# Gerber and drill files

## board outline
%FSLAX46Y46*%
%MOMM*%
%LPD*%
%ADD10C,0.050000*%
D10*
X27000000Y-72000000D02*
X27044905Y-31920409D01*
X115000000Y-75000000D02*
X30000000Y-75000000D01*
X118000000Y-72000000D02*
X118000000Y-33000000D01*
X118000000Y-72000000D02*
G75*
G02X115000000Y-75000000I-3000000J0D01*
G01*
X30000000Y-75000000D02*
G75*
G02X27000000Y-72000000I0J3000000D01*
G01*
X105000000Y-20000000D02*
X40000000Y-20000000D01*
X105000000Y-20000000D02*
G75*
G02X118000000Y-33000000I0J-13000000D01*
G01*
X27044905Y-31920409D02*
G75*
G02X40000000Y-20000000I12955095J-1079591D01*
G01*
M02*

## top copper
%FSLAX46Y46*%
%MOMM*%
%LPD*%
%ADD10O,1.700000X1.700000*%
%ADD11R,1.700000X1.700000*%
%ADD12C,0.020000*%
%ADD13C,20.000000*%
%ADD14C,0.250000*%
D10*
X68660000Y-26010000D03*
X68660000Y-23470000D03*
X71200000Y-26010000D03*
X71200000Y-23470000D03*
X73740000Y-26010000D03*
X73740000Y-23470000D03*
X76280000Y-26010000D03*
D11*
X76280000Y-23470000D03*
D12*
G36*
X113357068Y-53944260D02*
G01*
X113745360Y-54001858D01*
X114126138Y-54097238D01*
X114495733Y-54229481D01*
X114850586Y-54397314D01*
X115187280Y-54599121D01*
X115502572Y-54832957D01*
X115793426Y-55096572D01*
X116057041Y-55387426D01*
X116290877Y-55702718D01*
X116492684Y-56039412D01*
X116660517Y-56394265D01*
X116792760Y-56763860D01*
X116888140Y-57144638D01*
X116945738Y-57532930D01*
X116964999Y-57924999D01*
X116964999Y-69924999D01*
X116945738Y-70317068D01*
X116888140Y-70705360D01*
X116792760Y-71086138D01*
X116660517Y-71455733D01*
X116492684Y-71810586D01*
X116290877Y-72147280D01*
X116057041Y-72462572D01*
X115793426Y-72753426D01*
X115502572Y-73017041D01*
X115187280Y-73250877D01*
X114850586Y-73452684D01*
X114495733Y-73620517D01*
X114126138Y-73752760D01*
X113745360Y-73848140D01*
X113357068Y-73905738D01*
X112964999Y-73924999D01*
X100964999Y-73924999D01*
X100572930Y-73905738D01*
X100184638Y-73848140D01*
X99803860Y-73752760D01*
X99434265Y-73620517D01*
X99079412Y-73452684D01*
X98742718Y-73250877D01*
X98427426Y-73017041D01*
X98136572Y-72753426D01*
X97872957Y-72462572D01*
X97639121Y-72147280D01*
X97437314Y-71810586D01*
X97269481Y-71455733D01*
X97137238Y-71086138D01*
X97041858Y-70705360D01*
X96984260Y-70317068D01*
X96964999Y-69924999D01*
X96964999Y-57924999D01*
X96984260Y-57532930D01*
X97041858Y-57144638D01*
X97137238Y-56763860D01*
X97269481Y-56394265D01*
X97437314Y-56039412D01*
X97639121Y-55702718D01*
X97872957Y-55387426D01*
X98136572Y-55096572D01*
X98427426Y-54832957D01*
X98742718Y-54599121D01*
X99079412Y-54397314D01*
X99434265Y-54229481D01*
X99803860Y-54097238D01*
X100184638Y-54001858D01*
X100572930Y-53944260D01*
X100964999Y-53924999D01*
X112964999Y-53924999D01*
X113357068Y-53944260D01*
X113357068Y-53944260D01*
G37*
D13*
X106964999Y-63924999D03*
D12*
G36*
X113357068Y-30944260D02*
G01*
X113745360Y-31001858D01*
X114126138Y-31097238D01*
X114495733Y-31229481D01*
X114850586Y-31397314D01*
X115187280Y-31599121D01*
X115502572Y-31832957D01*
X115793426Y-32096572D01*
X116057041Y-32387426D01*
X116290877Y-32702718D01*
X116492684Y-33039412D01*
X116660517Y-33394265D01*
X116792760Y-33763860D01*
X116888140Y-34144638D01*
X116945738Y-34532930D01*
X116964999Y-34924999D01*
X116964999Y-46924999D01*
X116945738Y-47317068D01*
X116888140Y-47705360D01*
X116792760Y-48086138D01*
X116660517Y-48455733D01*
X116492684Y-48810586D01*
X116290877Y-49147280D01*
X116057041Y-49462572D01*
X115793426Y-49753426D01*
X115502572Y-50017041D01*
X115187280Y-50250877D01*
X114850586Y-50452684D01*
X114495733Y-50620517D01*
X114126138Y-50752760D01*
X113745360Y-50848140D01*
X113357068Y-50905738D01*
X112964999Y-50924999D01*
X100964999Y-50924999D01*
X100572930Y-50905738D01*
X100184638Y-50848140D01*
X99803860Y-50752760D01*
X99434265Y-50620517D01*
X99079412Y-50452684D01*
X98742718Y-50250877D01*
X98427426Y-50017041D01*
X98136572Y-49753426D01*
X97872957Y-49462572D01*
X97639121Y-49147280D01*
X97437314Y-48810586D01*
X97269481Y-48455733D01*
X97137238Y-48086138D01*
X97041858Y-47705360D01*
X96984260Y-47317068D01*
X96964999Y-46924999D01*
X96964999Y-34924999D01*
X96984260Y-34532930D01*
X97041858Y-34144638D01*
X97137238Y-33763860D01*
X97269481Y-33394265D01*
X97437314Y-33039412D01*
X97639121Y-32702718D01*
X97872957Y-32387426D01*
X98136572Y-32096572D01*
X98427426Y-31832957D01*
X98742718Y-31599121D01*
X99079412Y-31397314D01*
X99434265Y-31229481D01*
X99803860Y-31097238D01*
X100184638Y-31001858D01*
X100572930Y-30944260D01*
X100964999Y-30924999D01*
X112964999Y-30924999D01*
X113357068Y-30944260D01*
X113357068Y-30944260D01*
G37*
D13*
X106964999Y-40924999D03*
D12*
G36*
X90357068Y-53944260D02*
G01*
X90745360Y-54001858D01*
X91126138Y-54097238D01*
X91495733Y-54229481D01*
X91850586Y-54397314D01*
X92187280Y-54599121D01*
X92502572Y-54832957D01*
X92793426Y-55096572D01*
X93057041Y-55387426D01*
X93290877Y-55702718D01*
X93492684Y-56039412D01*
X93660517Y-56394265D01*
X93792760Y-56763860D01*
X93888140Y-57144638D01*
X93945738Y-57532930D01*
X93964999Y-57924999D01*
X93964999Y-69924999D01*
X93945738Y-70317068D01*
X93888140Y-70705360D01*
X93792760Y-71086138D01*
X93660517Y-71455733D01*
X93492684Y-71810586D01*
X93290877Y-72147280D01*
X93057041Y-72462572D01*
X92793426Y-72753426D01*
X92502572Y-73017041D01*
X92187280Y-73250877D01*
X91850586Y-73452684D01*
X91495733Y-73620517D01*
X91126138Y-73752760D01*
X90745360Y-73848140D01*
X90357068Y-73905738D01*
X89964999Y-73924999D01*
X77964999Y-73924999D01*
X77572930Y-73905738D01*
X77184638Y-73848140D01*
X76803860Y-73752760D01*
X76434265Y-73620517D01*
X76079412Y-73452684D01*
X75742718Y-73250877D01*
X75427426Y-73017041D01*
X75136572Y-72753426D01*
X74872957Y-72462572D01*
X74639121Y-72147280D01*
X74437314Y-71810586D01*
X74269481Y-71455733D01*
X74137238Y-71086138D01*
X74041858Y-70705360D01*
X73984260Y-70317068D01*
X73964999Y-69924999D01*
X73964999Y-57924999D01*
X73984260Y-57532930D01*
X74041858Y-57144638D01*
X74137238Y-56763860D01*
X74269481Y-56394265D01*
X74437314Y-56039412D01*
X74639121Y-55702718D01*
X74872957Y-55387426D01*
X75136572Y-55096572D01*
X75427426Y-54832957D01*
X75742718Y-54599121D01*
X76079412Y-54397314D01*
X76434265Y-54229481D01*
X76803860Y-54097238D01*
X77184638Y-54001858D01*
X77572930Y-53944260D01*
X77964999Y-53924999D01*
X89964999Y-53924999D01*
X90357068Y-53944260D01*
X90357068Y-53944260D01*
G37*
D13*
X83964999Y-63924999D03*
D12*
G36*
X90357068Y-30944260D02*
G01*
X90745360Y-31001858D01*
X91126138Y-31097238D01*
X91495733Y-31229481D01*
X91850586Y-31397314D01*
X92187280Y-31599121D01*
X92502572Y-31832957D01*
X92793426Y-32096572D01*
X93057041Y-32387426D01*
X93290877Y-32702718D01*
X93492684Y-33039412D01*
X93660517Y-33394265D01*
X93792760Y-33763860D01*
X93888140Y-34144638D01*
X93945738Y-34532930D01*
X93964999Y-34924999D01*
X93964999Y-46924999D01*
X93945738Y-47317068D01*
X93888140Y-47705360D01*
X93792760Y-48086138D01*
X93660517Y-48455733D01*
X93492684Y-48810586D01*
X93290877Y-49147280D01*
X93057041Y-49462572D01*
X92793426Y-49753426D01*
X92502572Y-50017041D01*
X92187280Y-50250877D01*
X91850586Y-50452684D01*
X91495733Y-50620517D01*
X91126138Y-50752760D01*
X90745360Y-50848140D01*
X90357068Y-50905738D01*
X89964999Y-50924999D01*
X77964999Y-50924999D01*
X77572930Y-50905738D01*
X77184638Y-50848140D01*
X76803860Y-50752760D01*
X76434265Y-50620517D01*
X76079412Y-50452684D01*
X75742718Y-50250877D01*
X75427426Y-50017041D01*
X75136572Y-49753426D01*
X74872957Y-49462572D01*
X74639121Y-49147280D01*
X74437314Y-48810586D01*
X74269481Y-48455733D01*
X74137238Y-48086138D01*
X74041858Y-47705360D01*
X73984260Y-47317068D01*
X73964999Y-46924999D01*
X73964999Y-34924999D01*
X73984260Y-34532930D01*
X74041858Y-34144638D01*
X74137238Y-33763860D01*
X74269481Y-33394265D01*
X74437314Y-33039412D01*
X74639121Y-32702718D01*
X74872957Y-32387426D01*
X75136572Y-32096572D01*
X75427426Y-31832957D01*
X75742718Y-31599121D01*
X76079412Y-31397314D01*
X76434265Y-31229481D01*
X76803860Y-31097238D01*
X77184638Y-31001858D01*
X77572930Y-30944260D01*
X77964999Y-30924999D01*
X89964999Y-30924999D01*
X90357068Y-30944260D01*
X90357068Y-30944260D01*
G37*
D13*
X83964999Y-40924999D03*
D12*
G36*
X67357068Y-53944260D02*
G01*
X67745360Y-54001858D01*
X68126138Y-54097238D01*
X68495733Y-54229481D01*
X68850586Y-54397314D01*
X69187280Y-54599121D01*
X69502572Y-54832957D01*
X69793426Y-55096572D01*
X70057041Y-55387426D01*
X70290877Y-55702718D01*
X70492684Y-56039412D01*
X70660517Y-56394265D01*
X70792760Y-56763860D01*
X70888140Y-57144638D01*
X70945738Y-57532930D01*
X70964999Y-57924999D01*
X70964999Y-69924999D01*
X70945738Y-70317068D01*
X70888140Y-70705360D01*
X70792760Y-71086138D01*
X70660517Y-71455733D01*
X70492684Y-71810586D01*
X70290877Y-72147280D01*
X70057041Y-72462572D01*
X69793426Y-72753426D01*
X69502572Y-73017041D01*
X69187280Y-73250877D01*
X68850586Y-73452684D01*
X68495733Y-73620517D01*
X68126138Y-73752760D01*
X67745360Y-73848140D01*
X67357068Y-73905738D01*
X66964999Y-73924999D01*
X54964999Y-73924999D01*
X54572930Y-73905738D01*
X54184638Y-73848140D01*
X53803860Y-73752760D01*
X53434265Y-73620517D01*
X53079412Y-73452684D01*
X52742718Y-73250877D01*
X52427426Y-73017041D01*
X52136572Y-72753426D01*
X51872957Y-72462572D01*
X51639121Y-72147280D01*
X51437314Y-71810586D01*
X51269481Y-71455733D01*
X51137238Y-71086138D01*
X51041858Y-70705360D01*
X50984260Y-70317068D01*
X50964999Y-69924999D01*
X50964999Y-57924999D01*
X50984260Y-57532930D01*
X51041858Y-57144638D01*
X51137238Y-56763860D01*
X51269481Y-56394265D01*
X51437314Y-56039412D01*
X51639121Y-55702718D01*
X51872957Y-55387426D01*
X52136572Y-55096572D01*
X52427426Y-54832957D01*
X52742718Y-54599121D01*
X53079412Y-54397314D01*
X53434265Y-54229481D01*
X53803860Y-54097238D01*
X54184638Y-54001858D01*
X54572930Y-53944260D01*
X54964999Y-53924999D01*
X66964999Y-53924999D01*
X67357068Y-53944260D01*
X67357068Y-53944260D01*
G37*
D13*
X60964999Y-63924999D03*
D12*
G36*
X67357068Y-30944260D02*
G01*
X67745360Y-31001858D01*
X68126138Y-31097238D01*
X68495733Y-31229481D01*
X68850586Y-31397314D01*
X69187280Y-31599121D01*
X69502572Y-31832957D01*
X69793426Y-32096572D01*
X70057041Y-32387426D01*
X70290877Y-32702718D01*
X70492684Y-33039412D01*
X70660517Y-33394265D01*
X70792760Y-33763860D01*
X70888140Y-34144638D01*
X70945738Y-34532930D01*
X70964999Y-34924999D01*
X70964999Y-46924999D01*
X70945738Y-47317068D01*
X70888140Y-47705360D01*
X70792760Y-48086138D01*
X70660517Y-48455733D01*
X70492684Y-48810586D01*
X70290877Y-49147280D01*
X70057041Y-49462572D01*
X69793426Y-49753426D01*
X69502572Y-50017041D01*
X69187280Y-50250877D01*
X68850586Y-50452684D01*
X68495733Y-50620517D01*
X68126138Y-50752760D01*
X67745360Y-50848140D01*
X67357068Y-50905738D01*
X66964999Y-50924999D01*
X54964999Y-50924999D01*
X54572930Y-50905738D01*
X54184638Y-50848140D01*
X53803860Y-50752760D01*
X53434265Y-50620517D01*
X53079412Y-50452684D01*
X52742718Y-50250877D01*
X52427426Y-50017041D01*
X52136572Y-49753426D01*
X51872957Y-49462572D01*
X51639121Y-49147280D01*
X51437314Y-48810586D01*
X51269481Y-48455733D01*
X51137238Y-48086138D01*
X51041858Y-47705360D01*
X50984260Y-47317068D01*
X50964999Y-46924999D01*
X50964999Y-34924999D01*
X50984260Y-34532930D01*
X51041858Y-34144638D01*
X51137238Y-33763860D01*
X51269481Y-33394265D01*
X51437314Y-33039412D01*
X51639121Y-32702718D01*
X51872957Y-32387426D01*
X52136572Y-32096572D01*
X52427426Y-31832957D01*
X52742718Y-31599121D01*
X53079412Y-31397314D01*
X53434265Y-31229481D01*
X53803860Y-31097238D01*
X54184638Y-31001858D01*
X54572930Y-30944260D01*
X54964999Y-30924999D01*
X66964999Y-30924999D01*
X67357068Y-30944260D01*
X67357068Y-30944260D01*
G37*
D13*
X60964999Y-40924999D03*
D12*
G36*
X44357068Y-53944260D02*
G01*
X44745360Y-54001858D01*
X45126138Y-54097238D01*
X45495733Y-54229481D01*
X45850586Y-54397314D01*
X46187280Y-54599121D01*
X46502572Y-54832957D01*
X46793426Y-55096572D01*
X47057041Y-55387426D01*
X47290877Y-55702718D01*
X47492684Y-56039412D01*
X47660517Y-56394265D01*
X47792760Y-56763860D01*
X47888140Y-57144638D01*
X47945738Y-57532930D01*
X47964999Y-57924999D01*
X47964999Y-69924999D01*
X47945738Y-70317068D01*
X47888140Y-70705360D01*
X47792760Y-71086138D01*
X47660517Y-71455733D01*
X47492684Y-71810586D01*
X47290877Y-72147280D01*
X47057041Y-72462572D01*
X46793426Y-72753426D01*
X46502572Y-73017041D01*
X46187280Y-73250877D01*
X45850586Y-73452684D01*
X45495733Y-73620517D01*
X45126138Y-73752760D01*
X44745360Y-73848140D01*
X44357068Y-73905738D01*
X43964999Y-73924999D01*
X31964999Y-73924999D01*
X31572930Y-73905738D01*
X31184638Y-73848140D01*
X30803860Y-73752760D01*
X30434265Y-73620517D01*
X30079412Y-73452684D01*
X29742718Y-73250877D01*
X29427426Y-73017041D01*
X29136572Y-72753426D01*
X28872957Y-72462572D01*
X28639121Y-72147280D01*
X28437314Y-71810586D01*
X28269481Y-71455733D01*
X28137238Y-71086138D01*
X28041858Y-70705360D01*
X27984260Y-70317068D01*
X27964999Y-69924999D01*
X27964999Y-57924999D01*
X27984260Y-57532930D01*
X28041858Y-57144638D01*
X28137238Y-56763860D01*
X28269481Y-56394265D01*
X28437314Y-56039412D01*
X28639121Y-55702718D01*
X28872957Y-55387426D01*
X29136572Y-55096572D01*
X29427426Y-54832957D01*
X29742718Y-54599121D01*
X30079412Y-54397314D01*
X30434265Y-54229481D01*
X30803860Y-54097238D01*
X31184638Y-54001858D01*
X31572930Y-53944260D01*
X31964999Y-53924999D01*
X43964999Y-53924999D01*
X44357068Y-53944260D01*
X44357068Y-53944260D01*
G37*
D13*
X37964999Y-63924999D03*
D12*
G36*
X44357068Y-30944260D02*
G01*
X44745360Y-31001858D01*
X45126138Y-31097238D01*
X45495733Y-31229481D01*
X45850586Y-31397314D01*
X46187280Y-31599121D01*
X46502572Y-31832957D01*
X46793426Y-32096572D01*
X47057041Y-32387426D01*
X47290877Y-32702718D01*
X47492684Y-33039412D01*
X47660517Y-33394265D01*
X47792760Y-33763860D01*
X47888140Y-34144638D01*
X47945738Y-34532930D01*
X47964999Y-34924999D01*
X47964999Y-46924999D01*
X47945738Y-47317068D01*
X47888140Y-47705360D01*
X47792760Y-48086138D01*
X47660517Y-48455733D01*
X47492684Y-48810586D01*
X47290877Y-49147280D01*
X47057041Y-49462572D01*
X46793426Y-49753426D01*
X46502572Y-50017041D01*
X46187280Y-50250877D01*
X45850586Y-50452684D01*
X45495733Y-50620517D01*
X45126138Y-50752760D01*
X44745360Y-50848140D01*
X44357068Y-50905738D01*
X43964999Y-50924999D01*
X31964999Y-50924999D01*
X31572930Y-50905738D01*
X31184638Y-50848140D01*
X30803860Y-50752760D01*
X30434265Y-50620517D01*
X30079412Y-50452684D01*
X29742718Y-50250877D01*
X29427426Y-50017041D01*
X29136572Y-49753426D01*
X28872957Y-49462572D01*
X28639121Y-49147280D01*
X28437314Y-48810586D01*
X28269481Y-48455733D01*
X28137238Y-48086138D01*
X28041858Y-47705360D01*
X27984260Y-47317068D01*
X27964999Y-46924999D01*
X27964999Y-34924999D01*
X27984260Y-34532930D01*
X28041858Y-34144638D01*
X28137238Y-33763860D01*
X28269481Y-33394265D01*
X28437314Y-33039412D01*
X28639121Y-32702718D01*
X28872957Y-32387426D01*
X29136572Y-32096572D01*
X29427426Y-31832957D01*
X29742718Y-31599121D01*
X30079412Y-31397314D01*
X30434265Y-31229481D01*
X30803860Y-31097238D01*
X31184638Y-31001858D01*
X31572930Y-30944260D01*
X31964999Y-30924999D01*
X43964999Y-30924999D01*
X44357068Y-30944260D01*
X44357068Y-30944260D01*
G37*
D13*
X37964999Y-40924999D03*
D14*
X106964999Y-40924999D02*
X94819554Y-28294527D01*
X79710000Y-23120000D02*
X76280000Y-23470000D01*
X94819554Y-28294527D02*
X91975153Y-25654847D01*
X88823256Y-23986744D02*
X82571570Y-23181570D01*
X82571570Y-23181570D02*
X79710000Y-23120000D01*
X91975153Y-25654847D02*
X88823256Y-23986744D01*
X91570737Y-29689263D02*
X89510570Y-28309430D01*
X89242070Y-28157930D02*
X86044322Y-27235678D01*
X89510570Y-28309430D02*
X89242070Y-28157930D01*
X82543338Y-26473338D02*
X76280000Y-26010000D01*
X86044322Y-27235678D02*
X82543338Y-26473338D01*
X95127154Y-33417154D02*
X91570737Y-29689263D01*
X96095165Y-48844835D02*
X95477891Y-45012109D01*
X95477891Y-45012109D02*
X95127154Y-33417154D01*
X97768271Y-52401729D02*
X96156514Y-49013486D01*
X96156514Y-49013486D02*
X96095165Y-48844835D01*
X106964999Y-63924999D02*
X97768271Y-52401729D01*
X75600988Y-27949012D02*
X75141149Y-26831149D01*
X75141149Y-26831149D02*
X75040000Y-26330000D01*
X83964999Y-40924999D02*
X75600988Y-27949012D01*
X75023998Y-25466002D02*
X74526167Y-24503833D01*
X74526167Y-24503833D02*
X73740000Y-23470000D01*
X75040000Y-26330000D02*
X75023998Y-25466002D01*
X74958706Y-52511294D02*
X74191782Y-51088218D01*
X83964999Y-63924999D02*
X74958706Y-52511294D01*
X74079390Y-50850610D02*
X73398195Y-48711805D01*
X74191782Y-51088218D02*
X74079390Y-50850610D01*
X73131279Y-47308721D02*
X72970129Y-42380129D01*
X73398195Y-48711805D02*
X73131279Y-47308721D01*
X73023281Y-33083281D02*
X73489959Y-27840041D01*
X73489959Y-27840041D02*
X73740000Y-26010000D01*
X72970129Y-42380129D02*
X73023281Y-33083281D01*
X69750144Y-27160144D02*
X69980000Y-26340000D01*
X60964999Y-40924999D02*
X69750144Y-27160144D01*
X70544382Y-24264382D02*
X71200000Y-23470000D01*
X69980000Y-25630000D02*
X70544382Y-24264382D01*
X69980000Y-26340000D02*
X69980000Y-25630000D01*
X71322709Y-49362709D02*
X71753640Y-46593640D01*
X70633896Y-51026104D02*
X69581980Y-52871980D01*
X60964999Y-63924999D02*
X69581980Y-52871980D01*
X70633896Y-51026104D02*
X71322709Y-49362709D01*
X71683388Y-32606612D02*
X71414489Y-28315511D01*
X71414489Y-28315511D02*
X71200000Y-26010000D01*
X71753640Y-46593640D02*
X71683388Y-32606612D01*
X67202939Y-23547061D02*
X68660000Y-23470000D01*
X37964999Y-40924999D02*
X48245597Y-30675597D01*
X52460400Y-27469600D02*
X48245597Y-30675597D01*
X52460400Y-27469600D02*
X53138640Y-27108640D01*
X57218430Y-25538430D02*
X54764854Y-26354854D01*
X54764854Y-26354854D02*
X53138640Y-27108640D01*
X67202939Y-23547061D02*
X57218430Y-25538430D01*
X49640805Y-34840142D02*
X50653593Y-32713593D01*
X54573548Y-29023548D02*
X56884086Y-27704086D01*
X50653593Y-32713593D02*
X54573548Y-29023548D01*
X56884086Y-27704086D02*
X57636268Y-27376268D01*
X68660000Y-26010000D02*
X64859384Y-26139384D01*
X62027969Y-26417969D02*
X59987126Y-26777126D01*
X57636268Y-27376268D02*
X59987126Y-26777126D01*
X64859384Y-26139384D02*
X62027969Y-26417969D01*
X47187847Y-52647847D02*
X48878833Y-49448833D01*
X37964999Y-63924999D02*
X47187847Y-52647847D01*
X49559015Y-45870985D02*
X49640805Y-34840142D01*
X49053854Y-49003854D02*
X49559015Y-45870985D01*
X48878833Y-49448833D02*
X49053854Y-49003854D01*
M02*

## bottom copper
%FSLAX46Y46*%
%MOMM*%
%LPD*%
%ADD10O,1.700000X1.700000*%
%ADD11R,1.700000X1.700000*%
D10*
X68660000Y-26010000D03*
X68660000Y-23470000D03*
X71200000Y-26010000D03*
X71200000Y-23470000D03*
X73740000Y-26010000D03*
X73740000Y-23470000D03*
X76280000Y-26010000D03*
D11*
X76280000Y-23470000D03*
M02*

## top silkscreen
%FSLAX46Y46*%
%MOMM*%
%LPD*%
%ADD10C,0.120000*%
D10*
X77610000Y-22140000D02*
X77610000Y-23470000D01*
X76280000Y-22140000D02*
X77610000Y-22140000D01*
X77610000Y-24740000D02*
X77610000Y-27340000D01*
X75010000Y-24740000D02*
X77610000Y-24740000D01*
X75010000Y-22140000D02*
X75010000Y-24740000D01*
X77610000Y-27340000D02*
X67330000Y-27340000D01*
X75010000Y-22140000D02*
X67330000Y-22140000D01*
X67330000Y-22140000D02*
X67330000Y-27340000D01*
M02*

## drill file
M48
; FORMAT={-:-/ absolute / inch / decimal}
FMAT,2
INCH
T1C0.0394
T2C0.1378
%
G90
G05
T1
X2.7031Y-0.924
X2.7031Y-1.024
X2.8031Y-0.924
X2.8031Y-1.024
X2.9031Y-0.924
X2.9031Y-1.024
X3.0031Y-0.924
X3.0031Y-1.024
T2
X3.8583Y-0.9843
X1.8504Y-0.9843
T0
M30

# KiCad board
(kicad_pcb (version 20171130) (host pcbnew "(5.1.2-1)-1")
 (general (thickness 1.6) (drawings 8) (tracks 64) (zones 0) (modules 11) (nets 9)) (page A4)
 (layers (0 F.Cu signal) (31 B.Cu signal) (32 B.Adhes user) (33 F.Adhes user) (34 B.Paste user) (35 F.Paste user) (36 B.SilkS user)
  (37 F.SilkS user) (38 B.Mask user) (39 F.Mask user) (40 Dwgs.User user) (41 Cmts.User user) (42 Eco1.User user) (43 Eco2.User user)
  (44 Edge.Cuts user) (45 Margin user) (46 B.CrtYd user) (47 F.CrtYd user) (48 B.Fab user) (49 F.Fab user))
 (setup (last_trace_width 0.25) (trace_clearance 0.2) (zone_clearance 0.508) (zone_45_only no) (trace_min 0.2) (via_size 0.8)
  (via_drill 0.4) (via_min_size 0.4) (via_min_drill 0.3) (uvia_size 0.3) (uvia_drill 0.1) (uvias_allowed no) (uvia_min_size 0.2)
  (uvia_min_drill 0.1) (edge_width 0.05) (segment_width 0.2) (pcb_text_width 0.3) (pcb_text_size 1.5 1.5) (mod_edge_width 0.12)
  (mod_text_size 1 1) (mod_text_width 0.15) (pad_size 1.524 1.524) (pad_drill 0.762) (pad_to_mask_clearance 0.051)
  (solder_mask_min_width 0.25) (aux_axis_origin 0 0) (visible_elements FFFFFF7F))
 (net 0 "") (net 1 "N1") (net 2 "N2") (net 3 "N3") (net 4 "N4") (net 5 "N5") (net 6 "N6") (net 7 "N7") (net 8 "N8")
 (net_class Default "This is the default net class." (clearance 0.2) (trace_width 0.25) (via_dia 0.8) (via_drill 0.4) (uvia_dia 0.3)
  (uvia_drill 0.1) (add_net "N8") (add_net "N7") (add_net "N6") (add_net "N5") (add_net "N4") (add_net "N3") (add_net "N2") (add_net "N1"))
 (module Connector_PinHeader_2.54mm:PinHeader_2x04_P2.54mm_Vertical (layer F.Cu) (at 76.28 23.47 270)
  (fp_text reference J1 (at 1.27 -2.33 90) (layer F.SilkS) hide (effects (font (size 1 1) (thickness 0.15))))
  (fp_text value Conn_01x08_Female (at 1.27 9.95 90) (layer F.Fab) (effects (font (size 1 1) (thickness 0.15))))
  (fp_line (start -1.33 -1.33) (end 0 -1.33) (layer F.SilkS) (width 0.12))
  (fp_line (start -1.33 0) (end -1.33 -1.33) (layer F.SilkS) (width 0.12))
  (fp_line (start 1.27 -1.33) (end 3.87 -1.33) (layer F.SilkS) (width 0.12))
  (fp_line (start 1.27 1.27) (end 1.27 -1.33) (layer F.SilkS) (width 0.12))
  (fp_line (start -1.33 1.27) (end 1.27 1.27) (layer F.SilkS) (width 0.12))
  (fp_line (start 3.87 -1.33) (end 3.87 8.95) (layer F.SilkS) (width 0.12))
  (fp_line (start -1.33 1.27) (end -1.33 8.95) (layer F.SilkS) (width 0.12))
  (fp_line (start -1.33 8.95) (end 3.87 8.95) (layer F.SilkS) (width 0.12))
  (pad 8 thru_hole oval (at 2.54 7.62 270) (size 1.7 1.7) (drill 1) (layers *.Cu *.Mask) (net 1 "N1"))
  (pad 7 thru_hole oval (at 0 7.62 270) (size 1.7 1.7) (drill 1) (layers *.Cu *.Mask) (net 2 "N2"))
  (pad 6 thru_hole oval (at 2.54 5.08 270) (size 1.7 1.7) (drill 1) (layers *.Cu *.Mask) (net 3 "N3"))
  (pad 5 thru_hole oval (at 0 5.08 270) (size 1.7 1.7) (drill 1) (layers *.Cu *.Mask) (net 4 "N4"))
  (pad 4 thru_hole oval (at 2.54 2.54 270) (size 1.7 1.7) (drill 1) (layers *.Cu *.Mask) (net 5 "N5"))
  (pad 3 thru_hole oval (at 0 2.54 270) (size 1.7 1.7) (drill 1) (layers *.Cu *.Mask) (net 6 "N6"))
  (pad 2 thru_hole oval (at 2.54 0 270) (size 1.7 1.7) (drill 1) (layers *.Cu *.Mask) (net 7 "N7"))
  (pad 1 thru_hole rect (at 0 0 270) (size 1.7 1.7) (drill 1) (layers *.Cu *.Mask) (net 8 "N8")))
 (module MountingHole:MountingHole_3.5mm (layer F.Cu) (at 98 25)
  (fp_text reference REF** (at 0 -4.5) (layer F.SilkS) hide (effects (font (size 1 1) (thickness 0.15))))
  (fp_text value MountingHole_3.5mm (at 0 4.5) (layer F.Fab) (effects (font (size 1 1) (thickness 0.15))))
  (pad 1 np_thru_hole circle (at 0 0) (size 3.5 3.5) (drill 3.5) (layers *.Cu *.Mask)))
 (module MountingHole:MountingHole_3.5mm (layer F.Cu) (at 47 25)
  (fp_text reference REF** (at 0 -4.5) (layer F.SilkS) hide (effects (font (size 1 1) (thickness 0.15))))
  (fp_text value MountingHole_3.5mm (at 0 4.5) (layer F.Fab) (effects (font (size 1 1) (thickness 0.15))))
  (pad 1 np_thru_hole circle (at 0 0) (size 3.5 3.5) (drill 3.5) (layers *.Cu *.Mask)))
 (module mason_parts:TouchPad (layer F.Cu) (at 106.984999 63.964999)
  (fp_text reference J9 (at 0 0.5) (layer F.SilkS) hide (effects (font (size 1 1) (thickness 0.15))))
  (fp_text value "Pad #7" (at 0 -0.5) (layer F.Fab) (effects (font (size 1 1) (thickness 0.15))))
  (pad 1 smd roundrect (at -0.02 -0.04) (size 20 20) (layers F.Cu F.Paste F.Mask) (roundrect_rratio 0.2) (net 7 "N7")))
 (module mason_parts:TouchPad (layer F.Cu) (at 106.984999 40.964999)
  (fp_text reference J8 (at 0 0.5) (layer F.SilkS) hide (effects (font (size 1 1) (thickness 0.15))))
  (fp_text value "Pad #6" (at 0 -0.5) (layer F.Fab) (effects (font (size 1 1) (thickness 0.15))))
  (pad 1 smd roundrect (at -0.02 -0.04) (size 20 20) (layers F.Cu F.Paste F.Mask) (roundrect_rratio 0.2) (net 8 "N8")))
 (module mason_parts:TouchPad (layer F.Cu) (at 83.984999 63.964999)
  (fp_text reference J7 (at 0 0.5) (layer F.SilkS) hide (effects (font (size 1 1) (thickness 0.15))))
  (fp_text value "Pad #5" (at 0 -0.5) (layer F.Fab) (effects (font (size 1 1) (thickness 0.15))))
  (pad 1 smd roundrect (at -0.02 -0.04) (size 20 20) (layers F.Cu F.Paste F.Mask) (roundrect_rratio 0.2) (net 5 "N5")))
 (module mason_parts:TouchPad (layer F.Cu) (at 83.984999 40.964999)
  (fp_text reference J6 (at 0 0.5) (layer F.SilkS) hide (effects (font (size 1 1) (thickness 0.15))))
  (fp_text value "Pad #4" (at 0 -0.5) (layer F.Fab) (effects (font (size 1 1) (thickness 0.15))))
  (pad 1 smd roundrect (at -0.02 -0.04) (size 20 20) (layers F.Cu F.Paste F.Mask) (roundrect_rratio 0.2) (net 6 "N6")))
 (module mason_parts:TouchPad (layer F.Cu) (at 60.984999 63.964999)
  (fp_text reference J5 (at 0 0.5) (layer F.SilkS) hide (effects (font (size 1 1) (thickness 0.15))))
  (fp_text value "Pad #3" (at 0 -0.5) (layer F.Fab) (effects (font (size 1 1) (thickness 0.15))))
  (pad 1 smd roundrect (at -0.02 -0.04) (size 20 20) (layers F.Cu F.Paste F.Mask) (roundrect_rratio 0.2) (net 3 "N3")))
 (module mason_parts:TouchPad (layer F.Cu) (at 60.984999 40.964999)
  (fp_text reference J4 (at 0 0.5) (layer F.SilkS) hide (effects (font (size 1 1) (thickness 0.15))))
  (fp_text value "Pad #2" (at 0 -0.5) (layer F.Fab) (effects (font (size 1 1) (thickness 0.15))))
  (pad 1 smd roundrect (at -0.02 -0.04) (size 20 20) (layers F.Cu F.Paste F.Mask) (roundrect_rratio 0.2) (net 4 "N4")))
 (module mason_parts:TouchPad (layer F.Cu) (at 37.984999 63.964999)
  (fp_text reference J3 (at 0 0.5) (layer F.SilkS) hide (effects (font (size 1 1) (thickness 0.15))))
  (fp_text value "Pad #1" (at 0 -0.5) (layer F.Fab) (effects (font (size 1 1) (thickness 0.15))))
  (pad 1 smd roundrect (at -0.02 -0.04) (size 20 20) (layers F.Cu F.Paste F.Mask) (roundrect_rratio 0.2) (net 1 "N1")))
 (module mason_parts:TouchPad (layer F.Cu) (at 37.984999 40.964999)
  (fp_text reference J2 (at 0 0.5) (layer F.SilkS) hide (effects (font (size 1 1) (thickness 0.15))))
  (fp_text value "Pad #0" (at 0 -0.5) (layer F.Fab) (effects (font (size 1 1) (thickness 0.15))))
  (pad 1 smd roundrect (at -0.02 -0.04) (size 20 20) (layers F.Cu F.Paste F.Mask) (roundrect_rratio 0.2) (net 2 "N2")))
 (gr_line (start 27 72) (end 27.044905 31.920409) (layer Edge.Cuts) (width 0.05))
 (gr_line (start 115 75) (end 30 75) (layer Edge.Cuts) (width 0.05))
 (gr_line (start 118 72) (end 118 33) (layer Edge.Cuts) (width 0.05))
 (gr_arc (start 115 72) (end 115 75) (angle -90) (layer Edge.Cuts) (width 0.05))
 (gr_arc (start 30 72) (end 27 72) (angle -90) (layer Edge.Cuts) (width 0.05))
 (gr_line (start 105 20) (end 40 20) (layer Edge.Cuts) (width 0.05))
 (gr_arc (start 105 33) (end 118 33) (angle -90) (layer Edge.Cuts) (width 0.05))
 (gr_arc (start 40 33) (end 40 20) (angle -85.23635831) (layer Edge.Cuts) (width 0.05))
 (segment (start 106.964999 40.924999) (end 94.819554 28.294527) (width 0.25) (layer F.Cu) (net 8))
 (segment (start 79.71 23.12) (end 76.28 23.47) (width 0.25) (layer F.Cu) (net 8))
 (segment (start 94.819554 28.294527) (end 91.975153 25.654847) (width 0.25) (layer F.Cu) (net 8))
 (segment (start 88.823256 23.986744) (end 82.57157 23.18157) (width 0.25) (layer F.Cu) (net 8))
 (segment (start 82.57157 23.18157) (end 79.71 23.12) (width 0.25) (layer F.Cu) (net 8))
 (segment (start 91.975153 25.654847) (end 88.823256 23.986744) (width 0.25) (layer F.Cu) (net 8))
 (segment (start 91.570737 29.689263) (end 89.51057 28.30943) (width 0.25) (layer F.Cu) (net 7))
 (segment (start 89.24207 28.15793) (end 86.044322 27.235678) (width 0.25) (layer F.Cu) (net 7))
 (segment (start 89.51057 28.30943) (end 89.24207 28.15793) (width 0.25) (layer F.Cu) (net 7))
 (segment (start 82.543338 26.473338) (end 76.28 26.01) (width 0.25) (layer F.Cu) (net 7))
 (segment (start 86.044322 27.235678) (end 82.543338 26.473338) (width 0.25) (layer F.Cu) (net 7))
 (segment (start 95.127154 33.417154) (end 91.570737 29.689263) (width 0.25) (layer F.Cu) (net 7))
 (segment (start 96.095165 48.844835) (end 95.477891 45.012109) (width 0.25) (layer F.Cu) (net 7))
 (segment (start 95.477891 45.012109) (end 95.127154 33.417154) (width 0.25) (layer F.Cu) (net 7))
 (segment (start 97.768271 52.401729) (end 96.156514 49.013486) (width 0.25) (layer F.Cu) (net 7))
 (segment (start 96.156514 49.013486) (end 96.095165 48.844835) (width 0.25) (layer F.Cu) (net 7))
 (segment (start 106.964999 63.924999) (end 97.768271 52.401729) (width 0.25) (layer F.Cu) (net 7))
 (segment (start 75.600988 27.949012) (end 75.141149 26.831149) (width 0.25) (layer F.Cu) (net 6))
 (segment (start 75.141149 26.831149) (end 75.04 26.33) (width 0.25) (layer F.Cu) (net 6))
 (segment (start 83.964999 40.924999) (end 75.600988 27.949012) (width 0.25) (layer F.Cu) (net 6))
 (segment (start 75.023998 25.466002) (end 74.526167 24.503833) (width 0.25) (layer F.Cu) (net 6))
 (segment (start 74.526167 24.503833) (end 73.74 23.47) (width 0.25) (layer F.Cu) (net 6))
 (segment (start 75.04 26.33) (end 75.023998 25.466002) (width 0.25) (layer F.Cu) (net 6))
 (segment (start 74.958706 52.511294) (end 74.191782 51.088218) (width 0.25) (layer F.Cu) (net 5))
 (segment (start 83.964999 63.924999) (end 74.958706 52.511294) (width 0.25) (layer F.Cu) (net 5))
 (segment (start 74.07939 50.85061) (end 73.398195 48.711805) (width 0.25) (layer F.Cu) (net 5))
 (segment (start 74.191782 51.088218) (end 74.07939 50.85061) (width 0.25) (layer F.Cu) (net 5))
 (segment (start 73.131279 47.308721) (end 72.970129 42.380129) (width 0.25) (layer F.Cu) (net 5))
 (segment (start 73.398195 48.711805) (end 73.131279 47.308721) (width 0.25) (layer F.Cu) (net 5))
 (segment (start 73.023281 33.083281) (end 73.489959 27.840041) (width 0.25) (layer F.Cu) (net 5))
 (segment (start 73.489959 27.840041) (end 73.74 26.01) (width 0.25) (layer F.Cu) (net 5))
 (segment (start 72.970129 42.380129) (end 73.023281 33.083281) (width 0.25) (layer F.Cu) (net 5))
 (segment (start 69.750144 27.160144) (end 69.98 26.34) (width 0.25) (layer F.Cu) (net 4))
 (segment (start 60.964999 40.924999) (end 69.750144 27.160144) (width 0.25) (layer F.Cu) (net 4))
 (segment (start 70.544382 24.264382) (end 71.2 23.47) (width 0.25) (layer F.Cu) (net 4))
 (segment (start 69.98 25.63) (end 70.544382 24.264382) (width 0.25) (layer F.Cu) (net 4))
 (segment (start 69.98 26.34) (end 69.98 25.63) (width 0.25) (layer F.Cu) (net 4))
 (segment (start 71.322709 49.362709) (end 71.75364 46.59364) (width 0.25) (layer F.Cu) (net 3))
 (segment (start 70.633896 51.026104) (end 69.58198 52.87198) (width 0.25) (layer F.Cu) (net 3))
 (segment (start 60.964999 63.924999) (end 69.58198 52.87198) (width 0.25) (layer F.Cu) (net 3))
 (segment (start 70.633896 51.026104) (end 71.322709 49.362709) (width 0.25) (layer F.Cu) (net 3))
 (segment (start 71.683388 32.606612) (end 71.414489 28.315511) (width 0.25) (layer F.Cu) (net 3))
 (segment (start 71.414489 28.315511) (end 71.2 26.01) (width 0.25) (layer F.Cu) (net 3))
 (segment (start 71.75364 46.59364) (end 71.683388 32.606612) (width 0.25) (layer F.Cu) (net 3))
 (segment (start 67.202939 23.547061) (end 68.66 23.47) (width 0.25) (layer F.Cu) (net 2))
 (segment (start 37.964999 40.924999) (end 48.245597 30.675597) (width 0.25) (layer F.Cu) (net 2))
 (segment (start 52.4604 27.4696) (end 48.245597 30.675597) (width 0.25) (layer F.Cu) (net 2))
 (segment (start 52.4604 27.4696) (end 53.13864 27.10864) (width 0.25) (layer F.Cu) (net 2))
 (segment (start 57.21843 25.53843) (end 54.764854 26.354854) (width 0.25) (layer F.Cu) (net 2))
 (segment (start 54.764854 26.354854) (end 53.13864 27.10864) (width 0.25) (layer F.Cu) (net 2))
 (segment (start 67.202939 23.547061) (end 57.21843 25.53843) (width 0.25) (layer F.Cu) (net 2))
 (segment (start 49.640805 34.840142) (end 50.653593 32.713593) (width 0.25) (layer F.Cu) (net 1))
 (segment (start 54.573548 29.023548) (end 56.884086 27.704086) (width 0.25) (layer F.Cu) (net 1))
 (segment (start 50.653593 32.713593) (end 54.573548 29.023548) (width 0.25) (layer F.Cu) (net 1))
 (segment (start 56.884086 27.704086) (end 57.636268 27.376268) (width 0.25) (layer F.Cu) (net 1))
 (segment (start 68.66 26.01) (end 64.859384 26.139384) (width 0.25) (layer F.Cu) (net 1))
 (segment (start 62.027969 26.417969) (end 59.987126 26.777126) (width 0.25) (layer F.Cu) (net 1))
 (segment (start 57.636268 27.376268) (end 59.987126 26.777126) (width 0.25) (layer F.Cu) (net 1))
 (segment (start 64.859384 26.139384) (end 62.027969 26.417969) (width 0.25) (layer F.Cu) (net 1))
 (segment (start 47.187847 52.647847) (end 48.878833 49.448833) (width 0.25) (layer F.Cu) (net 1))
 (segment (start 37.964999 63.924999) (end 47.187847 52.647847) (width 0.25) (layer F.Cu) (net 1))
 (segment (start 49.559015 45.870985) (end 49.640805 34.840142) (width 0.25) (layer F.Cu) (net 1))
 (segment (start 49.053854 49.003854) (end 49.559015 45.870985) (width 0.25) (layer F.Cu) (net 1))
 (segment (start 48.878833 49.448833) (end 49.053854 49.003854) (width 0.25) (layer F.Cu) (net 1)))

